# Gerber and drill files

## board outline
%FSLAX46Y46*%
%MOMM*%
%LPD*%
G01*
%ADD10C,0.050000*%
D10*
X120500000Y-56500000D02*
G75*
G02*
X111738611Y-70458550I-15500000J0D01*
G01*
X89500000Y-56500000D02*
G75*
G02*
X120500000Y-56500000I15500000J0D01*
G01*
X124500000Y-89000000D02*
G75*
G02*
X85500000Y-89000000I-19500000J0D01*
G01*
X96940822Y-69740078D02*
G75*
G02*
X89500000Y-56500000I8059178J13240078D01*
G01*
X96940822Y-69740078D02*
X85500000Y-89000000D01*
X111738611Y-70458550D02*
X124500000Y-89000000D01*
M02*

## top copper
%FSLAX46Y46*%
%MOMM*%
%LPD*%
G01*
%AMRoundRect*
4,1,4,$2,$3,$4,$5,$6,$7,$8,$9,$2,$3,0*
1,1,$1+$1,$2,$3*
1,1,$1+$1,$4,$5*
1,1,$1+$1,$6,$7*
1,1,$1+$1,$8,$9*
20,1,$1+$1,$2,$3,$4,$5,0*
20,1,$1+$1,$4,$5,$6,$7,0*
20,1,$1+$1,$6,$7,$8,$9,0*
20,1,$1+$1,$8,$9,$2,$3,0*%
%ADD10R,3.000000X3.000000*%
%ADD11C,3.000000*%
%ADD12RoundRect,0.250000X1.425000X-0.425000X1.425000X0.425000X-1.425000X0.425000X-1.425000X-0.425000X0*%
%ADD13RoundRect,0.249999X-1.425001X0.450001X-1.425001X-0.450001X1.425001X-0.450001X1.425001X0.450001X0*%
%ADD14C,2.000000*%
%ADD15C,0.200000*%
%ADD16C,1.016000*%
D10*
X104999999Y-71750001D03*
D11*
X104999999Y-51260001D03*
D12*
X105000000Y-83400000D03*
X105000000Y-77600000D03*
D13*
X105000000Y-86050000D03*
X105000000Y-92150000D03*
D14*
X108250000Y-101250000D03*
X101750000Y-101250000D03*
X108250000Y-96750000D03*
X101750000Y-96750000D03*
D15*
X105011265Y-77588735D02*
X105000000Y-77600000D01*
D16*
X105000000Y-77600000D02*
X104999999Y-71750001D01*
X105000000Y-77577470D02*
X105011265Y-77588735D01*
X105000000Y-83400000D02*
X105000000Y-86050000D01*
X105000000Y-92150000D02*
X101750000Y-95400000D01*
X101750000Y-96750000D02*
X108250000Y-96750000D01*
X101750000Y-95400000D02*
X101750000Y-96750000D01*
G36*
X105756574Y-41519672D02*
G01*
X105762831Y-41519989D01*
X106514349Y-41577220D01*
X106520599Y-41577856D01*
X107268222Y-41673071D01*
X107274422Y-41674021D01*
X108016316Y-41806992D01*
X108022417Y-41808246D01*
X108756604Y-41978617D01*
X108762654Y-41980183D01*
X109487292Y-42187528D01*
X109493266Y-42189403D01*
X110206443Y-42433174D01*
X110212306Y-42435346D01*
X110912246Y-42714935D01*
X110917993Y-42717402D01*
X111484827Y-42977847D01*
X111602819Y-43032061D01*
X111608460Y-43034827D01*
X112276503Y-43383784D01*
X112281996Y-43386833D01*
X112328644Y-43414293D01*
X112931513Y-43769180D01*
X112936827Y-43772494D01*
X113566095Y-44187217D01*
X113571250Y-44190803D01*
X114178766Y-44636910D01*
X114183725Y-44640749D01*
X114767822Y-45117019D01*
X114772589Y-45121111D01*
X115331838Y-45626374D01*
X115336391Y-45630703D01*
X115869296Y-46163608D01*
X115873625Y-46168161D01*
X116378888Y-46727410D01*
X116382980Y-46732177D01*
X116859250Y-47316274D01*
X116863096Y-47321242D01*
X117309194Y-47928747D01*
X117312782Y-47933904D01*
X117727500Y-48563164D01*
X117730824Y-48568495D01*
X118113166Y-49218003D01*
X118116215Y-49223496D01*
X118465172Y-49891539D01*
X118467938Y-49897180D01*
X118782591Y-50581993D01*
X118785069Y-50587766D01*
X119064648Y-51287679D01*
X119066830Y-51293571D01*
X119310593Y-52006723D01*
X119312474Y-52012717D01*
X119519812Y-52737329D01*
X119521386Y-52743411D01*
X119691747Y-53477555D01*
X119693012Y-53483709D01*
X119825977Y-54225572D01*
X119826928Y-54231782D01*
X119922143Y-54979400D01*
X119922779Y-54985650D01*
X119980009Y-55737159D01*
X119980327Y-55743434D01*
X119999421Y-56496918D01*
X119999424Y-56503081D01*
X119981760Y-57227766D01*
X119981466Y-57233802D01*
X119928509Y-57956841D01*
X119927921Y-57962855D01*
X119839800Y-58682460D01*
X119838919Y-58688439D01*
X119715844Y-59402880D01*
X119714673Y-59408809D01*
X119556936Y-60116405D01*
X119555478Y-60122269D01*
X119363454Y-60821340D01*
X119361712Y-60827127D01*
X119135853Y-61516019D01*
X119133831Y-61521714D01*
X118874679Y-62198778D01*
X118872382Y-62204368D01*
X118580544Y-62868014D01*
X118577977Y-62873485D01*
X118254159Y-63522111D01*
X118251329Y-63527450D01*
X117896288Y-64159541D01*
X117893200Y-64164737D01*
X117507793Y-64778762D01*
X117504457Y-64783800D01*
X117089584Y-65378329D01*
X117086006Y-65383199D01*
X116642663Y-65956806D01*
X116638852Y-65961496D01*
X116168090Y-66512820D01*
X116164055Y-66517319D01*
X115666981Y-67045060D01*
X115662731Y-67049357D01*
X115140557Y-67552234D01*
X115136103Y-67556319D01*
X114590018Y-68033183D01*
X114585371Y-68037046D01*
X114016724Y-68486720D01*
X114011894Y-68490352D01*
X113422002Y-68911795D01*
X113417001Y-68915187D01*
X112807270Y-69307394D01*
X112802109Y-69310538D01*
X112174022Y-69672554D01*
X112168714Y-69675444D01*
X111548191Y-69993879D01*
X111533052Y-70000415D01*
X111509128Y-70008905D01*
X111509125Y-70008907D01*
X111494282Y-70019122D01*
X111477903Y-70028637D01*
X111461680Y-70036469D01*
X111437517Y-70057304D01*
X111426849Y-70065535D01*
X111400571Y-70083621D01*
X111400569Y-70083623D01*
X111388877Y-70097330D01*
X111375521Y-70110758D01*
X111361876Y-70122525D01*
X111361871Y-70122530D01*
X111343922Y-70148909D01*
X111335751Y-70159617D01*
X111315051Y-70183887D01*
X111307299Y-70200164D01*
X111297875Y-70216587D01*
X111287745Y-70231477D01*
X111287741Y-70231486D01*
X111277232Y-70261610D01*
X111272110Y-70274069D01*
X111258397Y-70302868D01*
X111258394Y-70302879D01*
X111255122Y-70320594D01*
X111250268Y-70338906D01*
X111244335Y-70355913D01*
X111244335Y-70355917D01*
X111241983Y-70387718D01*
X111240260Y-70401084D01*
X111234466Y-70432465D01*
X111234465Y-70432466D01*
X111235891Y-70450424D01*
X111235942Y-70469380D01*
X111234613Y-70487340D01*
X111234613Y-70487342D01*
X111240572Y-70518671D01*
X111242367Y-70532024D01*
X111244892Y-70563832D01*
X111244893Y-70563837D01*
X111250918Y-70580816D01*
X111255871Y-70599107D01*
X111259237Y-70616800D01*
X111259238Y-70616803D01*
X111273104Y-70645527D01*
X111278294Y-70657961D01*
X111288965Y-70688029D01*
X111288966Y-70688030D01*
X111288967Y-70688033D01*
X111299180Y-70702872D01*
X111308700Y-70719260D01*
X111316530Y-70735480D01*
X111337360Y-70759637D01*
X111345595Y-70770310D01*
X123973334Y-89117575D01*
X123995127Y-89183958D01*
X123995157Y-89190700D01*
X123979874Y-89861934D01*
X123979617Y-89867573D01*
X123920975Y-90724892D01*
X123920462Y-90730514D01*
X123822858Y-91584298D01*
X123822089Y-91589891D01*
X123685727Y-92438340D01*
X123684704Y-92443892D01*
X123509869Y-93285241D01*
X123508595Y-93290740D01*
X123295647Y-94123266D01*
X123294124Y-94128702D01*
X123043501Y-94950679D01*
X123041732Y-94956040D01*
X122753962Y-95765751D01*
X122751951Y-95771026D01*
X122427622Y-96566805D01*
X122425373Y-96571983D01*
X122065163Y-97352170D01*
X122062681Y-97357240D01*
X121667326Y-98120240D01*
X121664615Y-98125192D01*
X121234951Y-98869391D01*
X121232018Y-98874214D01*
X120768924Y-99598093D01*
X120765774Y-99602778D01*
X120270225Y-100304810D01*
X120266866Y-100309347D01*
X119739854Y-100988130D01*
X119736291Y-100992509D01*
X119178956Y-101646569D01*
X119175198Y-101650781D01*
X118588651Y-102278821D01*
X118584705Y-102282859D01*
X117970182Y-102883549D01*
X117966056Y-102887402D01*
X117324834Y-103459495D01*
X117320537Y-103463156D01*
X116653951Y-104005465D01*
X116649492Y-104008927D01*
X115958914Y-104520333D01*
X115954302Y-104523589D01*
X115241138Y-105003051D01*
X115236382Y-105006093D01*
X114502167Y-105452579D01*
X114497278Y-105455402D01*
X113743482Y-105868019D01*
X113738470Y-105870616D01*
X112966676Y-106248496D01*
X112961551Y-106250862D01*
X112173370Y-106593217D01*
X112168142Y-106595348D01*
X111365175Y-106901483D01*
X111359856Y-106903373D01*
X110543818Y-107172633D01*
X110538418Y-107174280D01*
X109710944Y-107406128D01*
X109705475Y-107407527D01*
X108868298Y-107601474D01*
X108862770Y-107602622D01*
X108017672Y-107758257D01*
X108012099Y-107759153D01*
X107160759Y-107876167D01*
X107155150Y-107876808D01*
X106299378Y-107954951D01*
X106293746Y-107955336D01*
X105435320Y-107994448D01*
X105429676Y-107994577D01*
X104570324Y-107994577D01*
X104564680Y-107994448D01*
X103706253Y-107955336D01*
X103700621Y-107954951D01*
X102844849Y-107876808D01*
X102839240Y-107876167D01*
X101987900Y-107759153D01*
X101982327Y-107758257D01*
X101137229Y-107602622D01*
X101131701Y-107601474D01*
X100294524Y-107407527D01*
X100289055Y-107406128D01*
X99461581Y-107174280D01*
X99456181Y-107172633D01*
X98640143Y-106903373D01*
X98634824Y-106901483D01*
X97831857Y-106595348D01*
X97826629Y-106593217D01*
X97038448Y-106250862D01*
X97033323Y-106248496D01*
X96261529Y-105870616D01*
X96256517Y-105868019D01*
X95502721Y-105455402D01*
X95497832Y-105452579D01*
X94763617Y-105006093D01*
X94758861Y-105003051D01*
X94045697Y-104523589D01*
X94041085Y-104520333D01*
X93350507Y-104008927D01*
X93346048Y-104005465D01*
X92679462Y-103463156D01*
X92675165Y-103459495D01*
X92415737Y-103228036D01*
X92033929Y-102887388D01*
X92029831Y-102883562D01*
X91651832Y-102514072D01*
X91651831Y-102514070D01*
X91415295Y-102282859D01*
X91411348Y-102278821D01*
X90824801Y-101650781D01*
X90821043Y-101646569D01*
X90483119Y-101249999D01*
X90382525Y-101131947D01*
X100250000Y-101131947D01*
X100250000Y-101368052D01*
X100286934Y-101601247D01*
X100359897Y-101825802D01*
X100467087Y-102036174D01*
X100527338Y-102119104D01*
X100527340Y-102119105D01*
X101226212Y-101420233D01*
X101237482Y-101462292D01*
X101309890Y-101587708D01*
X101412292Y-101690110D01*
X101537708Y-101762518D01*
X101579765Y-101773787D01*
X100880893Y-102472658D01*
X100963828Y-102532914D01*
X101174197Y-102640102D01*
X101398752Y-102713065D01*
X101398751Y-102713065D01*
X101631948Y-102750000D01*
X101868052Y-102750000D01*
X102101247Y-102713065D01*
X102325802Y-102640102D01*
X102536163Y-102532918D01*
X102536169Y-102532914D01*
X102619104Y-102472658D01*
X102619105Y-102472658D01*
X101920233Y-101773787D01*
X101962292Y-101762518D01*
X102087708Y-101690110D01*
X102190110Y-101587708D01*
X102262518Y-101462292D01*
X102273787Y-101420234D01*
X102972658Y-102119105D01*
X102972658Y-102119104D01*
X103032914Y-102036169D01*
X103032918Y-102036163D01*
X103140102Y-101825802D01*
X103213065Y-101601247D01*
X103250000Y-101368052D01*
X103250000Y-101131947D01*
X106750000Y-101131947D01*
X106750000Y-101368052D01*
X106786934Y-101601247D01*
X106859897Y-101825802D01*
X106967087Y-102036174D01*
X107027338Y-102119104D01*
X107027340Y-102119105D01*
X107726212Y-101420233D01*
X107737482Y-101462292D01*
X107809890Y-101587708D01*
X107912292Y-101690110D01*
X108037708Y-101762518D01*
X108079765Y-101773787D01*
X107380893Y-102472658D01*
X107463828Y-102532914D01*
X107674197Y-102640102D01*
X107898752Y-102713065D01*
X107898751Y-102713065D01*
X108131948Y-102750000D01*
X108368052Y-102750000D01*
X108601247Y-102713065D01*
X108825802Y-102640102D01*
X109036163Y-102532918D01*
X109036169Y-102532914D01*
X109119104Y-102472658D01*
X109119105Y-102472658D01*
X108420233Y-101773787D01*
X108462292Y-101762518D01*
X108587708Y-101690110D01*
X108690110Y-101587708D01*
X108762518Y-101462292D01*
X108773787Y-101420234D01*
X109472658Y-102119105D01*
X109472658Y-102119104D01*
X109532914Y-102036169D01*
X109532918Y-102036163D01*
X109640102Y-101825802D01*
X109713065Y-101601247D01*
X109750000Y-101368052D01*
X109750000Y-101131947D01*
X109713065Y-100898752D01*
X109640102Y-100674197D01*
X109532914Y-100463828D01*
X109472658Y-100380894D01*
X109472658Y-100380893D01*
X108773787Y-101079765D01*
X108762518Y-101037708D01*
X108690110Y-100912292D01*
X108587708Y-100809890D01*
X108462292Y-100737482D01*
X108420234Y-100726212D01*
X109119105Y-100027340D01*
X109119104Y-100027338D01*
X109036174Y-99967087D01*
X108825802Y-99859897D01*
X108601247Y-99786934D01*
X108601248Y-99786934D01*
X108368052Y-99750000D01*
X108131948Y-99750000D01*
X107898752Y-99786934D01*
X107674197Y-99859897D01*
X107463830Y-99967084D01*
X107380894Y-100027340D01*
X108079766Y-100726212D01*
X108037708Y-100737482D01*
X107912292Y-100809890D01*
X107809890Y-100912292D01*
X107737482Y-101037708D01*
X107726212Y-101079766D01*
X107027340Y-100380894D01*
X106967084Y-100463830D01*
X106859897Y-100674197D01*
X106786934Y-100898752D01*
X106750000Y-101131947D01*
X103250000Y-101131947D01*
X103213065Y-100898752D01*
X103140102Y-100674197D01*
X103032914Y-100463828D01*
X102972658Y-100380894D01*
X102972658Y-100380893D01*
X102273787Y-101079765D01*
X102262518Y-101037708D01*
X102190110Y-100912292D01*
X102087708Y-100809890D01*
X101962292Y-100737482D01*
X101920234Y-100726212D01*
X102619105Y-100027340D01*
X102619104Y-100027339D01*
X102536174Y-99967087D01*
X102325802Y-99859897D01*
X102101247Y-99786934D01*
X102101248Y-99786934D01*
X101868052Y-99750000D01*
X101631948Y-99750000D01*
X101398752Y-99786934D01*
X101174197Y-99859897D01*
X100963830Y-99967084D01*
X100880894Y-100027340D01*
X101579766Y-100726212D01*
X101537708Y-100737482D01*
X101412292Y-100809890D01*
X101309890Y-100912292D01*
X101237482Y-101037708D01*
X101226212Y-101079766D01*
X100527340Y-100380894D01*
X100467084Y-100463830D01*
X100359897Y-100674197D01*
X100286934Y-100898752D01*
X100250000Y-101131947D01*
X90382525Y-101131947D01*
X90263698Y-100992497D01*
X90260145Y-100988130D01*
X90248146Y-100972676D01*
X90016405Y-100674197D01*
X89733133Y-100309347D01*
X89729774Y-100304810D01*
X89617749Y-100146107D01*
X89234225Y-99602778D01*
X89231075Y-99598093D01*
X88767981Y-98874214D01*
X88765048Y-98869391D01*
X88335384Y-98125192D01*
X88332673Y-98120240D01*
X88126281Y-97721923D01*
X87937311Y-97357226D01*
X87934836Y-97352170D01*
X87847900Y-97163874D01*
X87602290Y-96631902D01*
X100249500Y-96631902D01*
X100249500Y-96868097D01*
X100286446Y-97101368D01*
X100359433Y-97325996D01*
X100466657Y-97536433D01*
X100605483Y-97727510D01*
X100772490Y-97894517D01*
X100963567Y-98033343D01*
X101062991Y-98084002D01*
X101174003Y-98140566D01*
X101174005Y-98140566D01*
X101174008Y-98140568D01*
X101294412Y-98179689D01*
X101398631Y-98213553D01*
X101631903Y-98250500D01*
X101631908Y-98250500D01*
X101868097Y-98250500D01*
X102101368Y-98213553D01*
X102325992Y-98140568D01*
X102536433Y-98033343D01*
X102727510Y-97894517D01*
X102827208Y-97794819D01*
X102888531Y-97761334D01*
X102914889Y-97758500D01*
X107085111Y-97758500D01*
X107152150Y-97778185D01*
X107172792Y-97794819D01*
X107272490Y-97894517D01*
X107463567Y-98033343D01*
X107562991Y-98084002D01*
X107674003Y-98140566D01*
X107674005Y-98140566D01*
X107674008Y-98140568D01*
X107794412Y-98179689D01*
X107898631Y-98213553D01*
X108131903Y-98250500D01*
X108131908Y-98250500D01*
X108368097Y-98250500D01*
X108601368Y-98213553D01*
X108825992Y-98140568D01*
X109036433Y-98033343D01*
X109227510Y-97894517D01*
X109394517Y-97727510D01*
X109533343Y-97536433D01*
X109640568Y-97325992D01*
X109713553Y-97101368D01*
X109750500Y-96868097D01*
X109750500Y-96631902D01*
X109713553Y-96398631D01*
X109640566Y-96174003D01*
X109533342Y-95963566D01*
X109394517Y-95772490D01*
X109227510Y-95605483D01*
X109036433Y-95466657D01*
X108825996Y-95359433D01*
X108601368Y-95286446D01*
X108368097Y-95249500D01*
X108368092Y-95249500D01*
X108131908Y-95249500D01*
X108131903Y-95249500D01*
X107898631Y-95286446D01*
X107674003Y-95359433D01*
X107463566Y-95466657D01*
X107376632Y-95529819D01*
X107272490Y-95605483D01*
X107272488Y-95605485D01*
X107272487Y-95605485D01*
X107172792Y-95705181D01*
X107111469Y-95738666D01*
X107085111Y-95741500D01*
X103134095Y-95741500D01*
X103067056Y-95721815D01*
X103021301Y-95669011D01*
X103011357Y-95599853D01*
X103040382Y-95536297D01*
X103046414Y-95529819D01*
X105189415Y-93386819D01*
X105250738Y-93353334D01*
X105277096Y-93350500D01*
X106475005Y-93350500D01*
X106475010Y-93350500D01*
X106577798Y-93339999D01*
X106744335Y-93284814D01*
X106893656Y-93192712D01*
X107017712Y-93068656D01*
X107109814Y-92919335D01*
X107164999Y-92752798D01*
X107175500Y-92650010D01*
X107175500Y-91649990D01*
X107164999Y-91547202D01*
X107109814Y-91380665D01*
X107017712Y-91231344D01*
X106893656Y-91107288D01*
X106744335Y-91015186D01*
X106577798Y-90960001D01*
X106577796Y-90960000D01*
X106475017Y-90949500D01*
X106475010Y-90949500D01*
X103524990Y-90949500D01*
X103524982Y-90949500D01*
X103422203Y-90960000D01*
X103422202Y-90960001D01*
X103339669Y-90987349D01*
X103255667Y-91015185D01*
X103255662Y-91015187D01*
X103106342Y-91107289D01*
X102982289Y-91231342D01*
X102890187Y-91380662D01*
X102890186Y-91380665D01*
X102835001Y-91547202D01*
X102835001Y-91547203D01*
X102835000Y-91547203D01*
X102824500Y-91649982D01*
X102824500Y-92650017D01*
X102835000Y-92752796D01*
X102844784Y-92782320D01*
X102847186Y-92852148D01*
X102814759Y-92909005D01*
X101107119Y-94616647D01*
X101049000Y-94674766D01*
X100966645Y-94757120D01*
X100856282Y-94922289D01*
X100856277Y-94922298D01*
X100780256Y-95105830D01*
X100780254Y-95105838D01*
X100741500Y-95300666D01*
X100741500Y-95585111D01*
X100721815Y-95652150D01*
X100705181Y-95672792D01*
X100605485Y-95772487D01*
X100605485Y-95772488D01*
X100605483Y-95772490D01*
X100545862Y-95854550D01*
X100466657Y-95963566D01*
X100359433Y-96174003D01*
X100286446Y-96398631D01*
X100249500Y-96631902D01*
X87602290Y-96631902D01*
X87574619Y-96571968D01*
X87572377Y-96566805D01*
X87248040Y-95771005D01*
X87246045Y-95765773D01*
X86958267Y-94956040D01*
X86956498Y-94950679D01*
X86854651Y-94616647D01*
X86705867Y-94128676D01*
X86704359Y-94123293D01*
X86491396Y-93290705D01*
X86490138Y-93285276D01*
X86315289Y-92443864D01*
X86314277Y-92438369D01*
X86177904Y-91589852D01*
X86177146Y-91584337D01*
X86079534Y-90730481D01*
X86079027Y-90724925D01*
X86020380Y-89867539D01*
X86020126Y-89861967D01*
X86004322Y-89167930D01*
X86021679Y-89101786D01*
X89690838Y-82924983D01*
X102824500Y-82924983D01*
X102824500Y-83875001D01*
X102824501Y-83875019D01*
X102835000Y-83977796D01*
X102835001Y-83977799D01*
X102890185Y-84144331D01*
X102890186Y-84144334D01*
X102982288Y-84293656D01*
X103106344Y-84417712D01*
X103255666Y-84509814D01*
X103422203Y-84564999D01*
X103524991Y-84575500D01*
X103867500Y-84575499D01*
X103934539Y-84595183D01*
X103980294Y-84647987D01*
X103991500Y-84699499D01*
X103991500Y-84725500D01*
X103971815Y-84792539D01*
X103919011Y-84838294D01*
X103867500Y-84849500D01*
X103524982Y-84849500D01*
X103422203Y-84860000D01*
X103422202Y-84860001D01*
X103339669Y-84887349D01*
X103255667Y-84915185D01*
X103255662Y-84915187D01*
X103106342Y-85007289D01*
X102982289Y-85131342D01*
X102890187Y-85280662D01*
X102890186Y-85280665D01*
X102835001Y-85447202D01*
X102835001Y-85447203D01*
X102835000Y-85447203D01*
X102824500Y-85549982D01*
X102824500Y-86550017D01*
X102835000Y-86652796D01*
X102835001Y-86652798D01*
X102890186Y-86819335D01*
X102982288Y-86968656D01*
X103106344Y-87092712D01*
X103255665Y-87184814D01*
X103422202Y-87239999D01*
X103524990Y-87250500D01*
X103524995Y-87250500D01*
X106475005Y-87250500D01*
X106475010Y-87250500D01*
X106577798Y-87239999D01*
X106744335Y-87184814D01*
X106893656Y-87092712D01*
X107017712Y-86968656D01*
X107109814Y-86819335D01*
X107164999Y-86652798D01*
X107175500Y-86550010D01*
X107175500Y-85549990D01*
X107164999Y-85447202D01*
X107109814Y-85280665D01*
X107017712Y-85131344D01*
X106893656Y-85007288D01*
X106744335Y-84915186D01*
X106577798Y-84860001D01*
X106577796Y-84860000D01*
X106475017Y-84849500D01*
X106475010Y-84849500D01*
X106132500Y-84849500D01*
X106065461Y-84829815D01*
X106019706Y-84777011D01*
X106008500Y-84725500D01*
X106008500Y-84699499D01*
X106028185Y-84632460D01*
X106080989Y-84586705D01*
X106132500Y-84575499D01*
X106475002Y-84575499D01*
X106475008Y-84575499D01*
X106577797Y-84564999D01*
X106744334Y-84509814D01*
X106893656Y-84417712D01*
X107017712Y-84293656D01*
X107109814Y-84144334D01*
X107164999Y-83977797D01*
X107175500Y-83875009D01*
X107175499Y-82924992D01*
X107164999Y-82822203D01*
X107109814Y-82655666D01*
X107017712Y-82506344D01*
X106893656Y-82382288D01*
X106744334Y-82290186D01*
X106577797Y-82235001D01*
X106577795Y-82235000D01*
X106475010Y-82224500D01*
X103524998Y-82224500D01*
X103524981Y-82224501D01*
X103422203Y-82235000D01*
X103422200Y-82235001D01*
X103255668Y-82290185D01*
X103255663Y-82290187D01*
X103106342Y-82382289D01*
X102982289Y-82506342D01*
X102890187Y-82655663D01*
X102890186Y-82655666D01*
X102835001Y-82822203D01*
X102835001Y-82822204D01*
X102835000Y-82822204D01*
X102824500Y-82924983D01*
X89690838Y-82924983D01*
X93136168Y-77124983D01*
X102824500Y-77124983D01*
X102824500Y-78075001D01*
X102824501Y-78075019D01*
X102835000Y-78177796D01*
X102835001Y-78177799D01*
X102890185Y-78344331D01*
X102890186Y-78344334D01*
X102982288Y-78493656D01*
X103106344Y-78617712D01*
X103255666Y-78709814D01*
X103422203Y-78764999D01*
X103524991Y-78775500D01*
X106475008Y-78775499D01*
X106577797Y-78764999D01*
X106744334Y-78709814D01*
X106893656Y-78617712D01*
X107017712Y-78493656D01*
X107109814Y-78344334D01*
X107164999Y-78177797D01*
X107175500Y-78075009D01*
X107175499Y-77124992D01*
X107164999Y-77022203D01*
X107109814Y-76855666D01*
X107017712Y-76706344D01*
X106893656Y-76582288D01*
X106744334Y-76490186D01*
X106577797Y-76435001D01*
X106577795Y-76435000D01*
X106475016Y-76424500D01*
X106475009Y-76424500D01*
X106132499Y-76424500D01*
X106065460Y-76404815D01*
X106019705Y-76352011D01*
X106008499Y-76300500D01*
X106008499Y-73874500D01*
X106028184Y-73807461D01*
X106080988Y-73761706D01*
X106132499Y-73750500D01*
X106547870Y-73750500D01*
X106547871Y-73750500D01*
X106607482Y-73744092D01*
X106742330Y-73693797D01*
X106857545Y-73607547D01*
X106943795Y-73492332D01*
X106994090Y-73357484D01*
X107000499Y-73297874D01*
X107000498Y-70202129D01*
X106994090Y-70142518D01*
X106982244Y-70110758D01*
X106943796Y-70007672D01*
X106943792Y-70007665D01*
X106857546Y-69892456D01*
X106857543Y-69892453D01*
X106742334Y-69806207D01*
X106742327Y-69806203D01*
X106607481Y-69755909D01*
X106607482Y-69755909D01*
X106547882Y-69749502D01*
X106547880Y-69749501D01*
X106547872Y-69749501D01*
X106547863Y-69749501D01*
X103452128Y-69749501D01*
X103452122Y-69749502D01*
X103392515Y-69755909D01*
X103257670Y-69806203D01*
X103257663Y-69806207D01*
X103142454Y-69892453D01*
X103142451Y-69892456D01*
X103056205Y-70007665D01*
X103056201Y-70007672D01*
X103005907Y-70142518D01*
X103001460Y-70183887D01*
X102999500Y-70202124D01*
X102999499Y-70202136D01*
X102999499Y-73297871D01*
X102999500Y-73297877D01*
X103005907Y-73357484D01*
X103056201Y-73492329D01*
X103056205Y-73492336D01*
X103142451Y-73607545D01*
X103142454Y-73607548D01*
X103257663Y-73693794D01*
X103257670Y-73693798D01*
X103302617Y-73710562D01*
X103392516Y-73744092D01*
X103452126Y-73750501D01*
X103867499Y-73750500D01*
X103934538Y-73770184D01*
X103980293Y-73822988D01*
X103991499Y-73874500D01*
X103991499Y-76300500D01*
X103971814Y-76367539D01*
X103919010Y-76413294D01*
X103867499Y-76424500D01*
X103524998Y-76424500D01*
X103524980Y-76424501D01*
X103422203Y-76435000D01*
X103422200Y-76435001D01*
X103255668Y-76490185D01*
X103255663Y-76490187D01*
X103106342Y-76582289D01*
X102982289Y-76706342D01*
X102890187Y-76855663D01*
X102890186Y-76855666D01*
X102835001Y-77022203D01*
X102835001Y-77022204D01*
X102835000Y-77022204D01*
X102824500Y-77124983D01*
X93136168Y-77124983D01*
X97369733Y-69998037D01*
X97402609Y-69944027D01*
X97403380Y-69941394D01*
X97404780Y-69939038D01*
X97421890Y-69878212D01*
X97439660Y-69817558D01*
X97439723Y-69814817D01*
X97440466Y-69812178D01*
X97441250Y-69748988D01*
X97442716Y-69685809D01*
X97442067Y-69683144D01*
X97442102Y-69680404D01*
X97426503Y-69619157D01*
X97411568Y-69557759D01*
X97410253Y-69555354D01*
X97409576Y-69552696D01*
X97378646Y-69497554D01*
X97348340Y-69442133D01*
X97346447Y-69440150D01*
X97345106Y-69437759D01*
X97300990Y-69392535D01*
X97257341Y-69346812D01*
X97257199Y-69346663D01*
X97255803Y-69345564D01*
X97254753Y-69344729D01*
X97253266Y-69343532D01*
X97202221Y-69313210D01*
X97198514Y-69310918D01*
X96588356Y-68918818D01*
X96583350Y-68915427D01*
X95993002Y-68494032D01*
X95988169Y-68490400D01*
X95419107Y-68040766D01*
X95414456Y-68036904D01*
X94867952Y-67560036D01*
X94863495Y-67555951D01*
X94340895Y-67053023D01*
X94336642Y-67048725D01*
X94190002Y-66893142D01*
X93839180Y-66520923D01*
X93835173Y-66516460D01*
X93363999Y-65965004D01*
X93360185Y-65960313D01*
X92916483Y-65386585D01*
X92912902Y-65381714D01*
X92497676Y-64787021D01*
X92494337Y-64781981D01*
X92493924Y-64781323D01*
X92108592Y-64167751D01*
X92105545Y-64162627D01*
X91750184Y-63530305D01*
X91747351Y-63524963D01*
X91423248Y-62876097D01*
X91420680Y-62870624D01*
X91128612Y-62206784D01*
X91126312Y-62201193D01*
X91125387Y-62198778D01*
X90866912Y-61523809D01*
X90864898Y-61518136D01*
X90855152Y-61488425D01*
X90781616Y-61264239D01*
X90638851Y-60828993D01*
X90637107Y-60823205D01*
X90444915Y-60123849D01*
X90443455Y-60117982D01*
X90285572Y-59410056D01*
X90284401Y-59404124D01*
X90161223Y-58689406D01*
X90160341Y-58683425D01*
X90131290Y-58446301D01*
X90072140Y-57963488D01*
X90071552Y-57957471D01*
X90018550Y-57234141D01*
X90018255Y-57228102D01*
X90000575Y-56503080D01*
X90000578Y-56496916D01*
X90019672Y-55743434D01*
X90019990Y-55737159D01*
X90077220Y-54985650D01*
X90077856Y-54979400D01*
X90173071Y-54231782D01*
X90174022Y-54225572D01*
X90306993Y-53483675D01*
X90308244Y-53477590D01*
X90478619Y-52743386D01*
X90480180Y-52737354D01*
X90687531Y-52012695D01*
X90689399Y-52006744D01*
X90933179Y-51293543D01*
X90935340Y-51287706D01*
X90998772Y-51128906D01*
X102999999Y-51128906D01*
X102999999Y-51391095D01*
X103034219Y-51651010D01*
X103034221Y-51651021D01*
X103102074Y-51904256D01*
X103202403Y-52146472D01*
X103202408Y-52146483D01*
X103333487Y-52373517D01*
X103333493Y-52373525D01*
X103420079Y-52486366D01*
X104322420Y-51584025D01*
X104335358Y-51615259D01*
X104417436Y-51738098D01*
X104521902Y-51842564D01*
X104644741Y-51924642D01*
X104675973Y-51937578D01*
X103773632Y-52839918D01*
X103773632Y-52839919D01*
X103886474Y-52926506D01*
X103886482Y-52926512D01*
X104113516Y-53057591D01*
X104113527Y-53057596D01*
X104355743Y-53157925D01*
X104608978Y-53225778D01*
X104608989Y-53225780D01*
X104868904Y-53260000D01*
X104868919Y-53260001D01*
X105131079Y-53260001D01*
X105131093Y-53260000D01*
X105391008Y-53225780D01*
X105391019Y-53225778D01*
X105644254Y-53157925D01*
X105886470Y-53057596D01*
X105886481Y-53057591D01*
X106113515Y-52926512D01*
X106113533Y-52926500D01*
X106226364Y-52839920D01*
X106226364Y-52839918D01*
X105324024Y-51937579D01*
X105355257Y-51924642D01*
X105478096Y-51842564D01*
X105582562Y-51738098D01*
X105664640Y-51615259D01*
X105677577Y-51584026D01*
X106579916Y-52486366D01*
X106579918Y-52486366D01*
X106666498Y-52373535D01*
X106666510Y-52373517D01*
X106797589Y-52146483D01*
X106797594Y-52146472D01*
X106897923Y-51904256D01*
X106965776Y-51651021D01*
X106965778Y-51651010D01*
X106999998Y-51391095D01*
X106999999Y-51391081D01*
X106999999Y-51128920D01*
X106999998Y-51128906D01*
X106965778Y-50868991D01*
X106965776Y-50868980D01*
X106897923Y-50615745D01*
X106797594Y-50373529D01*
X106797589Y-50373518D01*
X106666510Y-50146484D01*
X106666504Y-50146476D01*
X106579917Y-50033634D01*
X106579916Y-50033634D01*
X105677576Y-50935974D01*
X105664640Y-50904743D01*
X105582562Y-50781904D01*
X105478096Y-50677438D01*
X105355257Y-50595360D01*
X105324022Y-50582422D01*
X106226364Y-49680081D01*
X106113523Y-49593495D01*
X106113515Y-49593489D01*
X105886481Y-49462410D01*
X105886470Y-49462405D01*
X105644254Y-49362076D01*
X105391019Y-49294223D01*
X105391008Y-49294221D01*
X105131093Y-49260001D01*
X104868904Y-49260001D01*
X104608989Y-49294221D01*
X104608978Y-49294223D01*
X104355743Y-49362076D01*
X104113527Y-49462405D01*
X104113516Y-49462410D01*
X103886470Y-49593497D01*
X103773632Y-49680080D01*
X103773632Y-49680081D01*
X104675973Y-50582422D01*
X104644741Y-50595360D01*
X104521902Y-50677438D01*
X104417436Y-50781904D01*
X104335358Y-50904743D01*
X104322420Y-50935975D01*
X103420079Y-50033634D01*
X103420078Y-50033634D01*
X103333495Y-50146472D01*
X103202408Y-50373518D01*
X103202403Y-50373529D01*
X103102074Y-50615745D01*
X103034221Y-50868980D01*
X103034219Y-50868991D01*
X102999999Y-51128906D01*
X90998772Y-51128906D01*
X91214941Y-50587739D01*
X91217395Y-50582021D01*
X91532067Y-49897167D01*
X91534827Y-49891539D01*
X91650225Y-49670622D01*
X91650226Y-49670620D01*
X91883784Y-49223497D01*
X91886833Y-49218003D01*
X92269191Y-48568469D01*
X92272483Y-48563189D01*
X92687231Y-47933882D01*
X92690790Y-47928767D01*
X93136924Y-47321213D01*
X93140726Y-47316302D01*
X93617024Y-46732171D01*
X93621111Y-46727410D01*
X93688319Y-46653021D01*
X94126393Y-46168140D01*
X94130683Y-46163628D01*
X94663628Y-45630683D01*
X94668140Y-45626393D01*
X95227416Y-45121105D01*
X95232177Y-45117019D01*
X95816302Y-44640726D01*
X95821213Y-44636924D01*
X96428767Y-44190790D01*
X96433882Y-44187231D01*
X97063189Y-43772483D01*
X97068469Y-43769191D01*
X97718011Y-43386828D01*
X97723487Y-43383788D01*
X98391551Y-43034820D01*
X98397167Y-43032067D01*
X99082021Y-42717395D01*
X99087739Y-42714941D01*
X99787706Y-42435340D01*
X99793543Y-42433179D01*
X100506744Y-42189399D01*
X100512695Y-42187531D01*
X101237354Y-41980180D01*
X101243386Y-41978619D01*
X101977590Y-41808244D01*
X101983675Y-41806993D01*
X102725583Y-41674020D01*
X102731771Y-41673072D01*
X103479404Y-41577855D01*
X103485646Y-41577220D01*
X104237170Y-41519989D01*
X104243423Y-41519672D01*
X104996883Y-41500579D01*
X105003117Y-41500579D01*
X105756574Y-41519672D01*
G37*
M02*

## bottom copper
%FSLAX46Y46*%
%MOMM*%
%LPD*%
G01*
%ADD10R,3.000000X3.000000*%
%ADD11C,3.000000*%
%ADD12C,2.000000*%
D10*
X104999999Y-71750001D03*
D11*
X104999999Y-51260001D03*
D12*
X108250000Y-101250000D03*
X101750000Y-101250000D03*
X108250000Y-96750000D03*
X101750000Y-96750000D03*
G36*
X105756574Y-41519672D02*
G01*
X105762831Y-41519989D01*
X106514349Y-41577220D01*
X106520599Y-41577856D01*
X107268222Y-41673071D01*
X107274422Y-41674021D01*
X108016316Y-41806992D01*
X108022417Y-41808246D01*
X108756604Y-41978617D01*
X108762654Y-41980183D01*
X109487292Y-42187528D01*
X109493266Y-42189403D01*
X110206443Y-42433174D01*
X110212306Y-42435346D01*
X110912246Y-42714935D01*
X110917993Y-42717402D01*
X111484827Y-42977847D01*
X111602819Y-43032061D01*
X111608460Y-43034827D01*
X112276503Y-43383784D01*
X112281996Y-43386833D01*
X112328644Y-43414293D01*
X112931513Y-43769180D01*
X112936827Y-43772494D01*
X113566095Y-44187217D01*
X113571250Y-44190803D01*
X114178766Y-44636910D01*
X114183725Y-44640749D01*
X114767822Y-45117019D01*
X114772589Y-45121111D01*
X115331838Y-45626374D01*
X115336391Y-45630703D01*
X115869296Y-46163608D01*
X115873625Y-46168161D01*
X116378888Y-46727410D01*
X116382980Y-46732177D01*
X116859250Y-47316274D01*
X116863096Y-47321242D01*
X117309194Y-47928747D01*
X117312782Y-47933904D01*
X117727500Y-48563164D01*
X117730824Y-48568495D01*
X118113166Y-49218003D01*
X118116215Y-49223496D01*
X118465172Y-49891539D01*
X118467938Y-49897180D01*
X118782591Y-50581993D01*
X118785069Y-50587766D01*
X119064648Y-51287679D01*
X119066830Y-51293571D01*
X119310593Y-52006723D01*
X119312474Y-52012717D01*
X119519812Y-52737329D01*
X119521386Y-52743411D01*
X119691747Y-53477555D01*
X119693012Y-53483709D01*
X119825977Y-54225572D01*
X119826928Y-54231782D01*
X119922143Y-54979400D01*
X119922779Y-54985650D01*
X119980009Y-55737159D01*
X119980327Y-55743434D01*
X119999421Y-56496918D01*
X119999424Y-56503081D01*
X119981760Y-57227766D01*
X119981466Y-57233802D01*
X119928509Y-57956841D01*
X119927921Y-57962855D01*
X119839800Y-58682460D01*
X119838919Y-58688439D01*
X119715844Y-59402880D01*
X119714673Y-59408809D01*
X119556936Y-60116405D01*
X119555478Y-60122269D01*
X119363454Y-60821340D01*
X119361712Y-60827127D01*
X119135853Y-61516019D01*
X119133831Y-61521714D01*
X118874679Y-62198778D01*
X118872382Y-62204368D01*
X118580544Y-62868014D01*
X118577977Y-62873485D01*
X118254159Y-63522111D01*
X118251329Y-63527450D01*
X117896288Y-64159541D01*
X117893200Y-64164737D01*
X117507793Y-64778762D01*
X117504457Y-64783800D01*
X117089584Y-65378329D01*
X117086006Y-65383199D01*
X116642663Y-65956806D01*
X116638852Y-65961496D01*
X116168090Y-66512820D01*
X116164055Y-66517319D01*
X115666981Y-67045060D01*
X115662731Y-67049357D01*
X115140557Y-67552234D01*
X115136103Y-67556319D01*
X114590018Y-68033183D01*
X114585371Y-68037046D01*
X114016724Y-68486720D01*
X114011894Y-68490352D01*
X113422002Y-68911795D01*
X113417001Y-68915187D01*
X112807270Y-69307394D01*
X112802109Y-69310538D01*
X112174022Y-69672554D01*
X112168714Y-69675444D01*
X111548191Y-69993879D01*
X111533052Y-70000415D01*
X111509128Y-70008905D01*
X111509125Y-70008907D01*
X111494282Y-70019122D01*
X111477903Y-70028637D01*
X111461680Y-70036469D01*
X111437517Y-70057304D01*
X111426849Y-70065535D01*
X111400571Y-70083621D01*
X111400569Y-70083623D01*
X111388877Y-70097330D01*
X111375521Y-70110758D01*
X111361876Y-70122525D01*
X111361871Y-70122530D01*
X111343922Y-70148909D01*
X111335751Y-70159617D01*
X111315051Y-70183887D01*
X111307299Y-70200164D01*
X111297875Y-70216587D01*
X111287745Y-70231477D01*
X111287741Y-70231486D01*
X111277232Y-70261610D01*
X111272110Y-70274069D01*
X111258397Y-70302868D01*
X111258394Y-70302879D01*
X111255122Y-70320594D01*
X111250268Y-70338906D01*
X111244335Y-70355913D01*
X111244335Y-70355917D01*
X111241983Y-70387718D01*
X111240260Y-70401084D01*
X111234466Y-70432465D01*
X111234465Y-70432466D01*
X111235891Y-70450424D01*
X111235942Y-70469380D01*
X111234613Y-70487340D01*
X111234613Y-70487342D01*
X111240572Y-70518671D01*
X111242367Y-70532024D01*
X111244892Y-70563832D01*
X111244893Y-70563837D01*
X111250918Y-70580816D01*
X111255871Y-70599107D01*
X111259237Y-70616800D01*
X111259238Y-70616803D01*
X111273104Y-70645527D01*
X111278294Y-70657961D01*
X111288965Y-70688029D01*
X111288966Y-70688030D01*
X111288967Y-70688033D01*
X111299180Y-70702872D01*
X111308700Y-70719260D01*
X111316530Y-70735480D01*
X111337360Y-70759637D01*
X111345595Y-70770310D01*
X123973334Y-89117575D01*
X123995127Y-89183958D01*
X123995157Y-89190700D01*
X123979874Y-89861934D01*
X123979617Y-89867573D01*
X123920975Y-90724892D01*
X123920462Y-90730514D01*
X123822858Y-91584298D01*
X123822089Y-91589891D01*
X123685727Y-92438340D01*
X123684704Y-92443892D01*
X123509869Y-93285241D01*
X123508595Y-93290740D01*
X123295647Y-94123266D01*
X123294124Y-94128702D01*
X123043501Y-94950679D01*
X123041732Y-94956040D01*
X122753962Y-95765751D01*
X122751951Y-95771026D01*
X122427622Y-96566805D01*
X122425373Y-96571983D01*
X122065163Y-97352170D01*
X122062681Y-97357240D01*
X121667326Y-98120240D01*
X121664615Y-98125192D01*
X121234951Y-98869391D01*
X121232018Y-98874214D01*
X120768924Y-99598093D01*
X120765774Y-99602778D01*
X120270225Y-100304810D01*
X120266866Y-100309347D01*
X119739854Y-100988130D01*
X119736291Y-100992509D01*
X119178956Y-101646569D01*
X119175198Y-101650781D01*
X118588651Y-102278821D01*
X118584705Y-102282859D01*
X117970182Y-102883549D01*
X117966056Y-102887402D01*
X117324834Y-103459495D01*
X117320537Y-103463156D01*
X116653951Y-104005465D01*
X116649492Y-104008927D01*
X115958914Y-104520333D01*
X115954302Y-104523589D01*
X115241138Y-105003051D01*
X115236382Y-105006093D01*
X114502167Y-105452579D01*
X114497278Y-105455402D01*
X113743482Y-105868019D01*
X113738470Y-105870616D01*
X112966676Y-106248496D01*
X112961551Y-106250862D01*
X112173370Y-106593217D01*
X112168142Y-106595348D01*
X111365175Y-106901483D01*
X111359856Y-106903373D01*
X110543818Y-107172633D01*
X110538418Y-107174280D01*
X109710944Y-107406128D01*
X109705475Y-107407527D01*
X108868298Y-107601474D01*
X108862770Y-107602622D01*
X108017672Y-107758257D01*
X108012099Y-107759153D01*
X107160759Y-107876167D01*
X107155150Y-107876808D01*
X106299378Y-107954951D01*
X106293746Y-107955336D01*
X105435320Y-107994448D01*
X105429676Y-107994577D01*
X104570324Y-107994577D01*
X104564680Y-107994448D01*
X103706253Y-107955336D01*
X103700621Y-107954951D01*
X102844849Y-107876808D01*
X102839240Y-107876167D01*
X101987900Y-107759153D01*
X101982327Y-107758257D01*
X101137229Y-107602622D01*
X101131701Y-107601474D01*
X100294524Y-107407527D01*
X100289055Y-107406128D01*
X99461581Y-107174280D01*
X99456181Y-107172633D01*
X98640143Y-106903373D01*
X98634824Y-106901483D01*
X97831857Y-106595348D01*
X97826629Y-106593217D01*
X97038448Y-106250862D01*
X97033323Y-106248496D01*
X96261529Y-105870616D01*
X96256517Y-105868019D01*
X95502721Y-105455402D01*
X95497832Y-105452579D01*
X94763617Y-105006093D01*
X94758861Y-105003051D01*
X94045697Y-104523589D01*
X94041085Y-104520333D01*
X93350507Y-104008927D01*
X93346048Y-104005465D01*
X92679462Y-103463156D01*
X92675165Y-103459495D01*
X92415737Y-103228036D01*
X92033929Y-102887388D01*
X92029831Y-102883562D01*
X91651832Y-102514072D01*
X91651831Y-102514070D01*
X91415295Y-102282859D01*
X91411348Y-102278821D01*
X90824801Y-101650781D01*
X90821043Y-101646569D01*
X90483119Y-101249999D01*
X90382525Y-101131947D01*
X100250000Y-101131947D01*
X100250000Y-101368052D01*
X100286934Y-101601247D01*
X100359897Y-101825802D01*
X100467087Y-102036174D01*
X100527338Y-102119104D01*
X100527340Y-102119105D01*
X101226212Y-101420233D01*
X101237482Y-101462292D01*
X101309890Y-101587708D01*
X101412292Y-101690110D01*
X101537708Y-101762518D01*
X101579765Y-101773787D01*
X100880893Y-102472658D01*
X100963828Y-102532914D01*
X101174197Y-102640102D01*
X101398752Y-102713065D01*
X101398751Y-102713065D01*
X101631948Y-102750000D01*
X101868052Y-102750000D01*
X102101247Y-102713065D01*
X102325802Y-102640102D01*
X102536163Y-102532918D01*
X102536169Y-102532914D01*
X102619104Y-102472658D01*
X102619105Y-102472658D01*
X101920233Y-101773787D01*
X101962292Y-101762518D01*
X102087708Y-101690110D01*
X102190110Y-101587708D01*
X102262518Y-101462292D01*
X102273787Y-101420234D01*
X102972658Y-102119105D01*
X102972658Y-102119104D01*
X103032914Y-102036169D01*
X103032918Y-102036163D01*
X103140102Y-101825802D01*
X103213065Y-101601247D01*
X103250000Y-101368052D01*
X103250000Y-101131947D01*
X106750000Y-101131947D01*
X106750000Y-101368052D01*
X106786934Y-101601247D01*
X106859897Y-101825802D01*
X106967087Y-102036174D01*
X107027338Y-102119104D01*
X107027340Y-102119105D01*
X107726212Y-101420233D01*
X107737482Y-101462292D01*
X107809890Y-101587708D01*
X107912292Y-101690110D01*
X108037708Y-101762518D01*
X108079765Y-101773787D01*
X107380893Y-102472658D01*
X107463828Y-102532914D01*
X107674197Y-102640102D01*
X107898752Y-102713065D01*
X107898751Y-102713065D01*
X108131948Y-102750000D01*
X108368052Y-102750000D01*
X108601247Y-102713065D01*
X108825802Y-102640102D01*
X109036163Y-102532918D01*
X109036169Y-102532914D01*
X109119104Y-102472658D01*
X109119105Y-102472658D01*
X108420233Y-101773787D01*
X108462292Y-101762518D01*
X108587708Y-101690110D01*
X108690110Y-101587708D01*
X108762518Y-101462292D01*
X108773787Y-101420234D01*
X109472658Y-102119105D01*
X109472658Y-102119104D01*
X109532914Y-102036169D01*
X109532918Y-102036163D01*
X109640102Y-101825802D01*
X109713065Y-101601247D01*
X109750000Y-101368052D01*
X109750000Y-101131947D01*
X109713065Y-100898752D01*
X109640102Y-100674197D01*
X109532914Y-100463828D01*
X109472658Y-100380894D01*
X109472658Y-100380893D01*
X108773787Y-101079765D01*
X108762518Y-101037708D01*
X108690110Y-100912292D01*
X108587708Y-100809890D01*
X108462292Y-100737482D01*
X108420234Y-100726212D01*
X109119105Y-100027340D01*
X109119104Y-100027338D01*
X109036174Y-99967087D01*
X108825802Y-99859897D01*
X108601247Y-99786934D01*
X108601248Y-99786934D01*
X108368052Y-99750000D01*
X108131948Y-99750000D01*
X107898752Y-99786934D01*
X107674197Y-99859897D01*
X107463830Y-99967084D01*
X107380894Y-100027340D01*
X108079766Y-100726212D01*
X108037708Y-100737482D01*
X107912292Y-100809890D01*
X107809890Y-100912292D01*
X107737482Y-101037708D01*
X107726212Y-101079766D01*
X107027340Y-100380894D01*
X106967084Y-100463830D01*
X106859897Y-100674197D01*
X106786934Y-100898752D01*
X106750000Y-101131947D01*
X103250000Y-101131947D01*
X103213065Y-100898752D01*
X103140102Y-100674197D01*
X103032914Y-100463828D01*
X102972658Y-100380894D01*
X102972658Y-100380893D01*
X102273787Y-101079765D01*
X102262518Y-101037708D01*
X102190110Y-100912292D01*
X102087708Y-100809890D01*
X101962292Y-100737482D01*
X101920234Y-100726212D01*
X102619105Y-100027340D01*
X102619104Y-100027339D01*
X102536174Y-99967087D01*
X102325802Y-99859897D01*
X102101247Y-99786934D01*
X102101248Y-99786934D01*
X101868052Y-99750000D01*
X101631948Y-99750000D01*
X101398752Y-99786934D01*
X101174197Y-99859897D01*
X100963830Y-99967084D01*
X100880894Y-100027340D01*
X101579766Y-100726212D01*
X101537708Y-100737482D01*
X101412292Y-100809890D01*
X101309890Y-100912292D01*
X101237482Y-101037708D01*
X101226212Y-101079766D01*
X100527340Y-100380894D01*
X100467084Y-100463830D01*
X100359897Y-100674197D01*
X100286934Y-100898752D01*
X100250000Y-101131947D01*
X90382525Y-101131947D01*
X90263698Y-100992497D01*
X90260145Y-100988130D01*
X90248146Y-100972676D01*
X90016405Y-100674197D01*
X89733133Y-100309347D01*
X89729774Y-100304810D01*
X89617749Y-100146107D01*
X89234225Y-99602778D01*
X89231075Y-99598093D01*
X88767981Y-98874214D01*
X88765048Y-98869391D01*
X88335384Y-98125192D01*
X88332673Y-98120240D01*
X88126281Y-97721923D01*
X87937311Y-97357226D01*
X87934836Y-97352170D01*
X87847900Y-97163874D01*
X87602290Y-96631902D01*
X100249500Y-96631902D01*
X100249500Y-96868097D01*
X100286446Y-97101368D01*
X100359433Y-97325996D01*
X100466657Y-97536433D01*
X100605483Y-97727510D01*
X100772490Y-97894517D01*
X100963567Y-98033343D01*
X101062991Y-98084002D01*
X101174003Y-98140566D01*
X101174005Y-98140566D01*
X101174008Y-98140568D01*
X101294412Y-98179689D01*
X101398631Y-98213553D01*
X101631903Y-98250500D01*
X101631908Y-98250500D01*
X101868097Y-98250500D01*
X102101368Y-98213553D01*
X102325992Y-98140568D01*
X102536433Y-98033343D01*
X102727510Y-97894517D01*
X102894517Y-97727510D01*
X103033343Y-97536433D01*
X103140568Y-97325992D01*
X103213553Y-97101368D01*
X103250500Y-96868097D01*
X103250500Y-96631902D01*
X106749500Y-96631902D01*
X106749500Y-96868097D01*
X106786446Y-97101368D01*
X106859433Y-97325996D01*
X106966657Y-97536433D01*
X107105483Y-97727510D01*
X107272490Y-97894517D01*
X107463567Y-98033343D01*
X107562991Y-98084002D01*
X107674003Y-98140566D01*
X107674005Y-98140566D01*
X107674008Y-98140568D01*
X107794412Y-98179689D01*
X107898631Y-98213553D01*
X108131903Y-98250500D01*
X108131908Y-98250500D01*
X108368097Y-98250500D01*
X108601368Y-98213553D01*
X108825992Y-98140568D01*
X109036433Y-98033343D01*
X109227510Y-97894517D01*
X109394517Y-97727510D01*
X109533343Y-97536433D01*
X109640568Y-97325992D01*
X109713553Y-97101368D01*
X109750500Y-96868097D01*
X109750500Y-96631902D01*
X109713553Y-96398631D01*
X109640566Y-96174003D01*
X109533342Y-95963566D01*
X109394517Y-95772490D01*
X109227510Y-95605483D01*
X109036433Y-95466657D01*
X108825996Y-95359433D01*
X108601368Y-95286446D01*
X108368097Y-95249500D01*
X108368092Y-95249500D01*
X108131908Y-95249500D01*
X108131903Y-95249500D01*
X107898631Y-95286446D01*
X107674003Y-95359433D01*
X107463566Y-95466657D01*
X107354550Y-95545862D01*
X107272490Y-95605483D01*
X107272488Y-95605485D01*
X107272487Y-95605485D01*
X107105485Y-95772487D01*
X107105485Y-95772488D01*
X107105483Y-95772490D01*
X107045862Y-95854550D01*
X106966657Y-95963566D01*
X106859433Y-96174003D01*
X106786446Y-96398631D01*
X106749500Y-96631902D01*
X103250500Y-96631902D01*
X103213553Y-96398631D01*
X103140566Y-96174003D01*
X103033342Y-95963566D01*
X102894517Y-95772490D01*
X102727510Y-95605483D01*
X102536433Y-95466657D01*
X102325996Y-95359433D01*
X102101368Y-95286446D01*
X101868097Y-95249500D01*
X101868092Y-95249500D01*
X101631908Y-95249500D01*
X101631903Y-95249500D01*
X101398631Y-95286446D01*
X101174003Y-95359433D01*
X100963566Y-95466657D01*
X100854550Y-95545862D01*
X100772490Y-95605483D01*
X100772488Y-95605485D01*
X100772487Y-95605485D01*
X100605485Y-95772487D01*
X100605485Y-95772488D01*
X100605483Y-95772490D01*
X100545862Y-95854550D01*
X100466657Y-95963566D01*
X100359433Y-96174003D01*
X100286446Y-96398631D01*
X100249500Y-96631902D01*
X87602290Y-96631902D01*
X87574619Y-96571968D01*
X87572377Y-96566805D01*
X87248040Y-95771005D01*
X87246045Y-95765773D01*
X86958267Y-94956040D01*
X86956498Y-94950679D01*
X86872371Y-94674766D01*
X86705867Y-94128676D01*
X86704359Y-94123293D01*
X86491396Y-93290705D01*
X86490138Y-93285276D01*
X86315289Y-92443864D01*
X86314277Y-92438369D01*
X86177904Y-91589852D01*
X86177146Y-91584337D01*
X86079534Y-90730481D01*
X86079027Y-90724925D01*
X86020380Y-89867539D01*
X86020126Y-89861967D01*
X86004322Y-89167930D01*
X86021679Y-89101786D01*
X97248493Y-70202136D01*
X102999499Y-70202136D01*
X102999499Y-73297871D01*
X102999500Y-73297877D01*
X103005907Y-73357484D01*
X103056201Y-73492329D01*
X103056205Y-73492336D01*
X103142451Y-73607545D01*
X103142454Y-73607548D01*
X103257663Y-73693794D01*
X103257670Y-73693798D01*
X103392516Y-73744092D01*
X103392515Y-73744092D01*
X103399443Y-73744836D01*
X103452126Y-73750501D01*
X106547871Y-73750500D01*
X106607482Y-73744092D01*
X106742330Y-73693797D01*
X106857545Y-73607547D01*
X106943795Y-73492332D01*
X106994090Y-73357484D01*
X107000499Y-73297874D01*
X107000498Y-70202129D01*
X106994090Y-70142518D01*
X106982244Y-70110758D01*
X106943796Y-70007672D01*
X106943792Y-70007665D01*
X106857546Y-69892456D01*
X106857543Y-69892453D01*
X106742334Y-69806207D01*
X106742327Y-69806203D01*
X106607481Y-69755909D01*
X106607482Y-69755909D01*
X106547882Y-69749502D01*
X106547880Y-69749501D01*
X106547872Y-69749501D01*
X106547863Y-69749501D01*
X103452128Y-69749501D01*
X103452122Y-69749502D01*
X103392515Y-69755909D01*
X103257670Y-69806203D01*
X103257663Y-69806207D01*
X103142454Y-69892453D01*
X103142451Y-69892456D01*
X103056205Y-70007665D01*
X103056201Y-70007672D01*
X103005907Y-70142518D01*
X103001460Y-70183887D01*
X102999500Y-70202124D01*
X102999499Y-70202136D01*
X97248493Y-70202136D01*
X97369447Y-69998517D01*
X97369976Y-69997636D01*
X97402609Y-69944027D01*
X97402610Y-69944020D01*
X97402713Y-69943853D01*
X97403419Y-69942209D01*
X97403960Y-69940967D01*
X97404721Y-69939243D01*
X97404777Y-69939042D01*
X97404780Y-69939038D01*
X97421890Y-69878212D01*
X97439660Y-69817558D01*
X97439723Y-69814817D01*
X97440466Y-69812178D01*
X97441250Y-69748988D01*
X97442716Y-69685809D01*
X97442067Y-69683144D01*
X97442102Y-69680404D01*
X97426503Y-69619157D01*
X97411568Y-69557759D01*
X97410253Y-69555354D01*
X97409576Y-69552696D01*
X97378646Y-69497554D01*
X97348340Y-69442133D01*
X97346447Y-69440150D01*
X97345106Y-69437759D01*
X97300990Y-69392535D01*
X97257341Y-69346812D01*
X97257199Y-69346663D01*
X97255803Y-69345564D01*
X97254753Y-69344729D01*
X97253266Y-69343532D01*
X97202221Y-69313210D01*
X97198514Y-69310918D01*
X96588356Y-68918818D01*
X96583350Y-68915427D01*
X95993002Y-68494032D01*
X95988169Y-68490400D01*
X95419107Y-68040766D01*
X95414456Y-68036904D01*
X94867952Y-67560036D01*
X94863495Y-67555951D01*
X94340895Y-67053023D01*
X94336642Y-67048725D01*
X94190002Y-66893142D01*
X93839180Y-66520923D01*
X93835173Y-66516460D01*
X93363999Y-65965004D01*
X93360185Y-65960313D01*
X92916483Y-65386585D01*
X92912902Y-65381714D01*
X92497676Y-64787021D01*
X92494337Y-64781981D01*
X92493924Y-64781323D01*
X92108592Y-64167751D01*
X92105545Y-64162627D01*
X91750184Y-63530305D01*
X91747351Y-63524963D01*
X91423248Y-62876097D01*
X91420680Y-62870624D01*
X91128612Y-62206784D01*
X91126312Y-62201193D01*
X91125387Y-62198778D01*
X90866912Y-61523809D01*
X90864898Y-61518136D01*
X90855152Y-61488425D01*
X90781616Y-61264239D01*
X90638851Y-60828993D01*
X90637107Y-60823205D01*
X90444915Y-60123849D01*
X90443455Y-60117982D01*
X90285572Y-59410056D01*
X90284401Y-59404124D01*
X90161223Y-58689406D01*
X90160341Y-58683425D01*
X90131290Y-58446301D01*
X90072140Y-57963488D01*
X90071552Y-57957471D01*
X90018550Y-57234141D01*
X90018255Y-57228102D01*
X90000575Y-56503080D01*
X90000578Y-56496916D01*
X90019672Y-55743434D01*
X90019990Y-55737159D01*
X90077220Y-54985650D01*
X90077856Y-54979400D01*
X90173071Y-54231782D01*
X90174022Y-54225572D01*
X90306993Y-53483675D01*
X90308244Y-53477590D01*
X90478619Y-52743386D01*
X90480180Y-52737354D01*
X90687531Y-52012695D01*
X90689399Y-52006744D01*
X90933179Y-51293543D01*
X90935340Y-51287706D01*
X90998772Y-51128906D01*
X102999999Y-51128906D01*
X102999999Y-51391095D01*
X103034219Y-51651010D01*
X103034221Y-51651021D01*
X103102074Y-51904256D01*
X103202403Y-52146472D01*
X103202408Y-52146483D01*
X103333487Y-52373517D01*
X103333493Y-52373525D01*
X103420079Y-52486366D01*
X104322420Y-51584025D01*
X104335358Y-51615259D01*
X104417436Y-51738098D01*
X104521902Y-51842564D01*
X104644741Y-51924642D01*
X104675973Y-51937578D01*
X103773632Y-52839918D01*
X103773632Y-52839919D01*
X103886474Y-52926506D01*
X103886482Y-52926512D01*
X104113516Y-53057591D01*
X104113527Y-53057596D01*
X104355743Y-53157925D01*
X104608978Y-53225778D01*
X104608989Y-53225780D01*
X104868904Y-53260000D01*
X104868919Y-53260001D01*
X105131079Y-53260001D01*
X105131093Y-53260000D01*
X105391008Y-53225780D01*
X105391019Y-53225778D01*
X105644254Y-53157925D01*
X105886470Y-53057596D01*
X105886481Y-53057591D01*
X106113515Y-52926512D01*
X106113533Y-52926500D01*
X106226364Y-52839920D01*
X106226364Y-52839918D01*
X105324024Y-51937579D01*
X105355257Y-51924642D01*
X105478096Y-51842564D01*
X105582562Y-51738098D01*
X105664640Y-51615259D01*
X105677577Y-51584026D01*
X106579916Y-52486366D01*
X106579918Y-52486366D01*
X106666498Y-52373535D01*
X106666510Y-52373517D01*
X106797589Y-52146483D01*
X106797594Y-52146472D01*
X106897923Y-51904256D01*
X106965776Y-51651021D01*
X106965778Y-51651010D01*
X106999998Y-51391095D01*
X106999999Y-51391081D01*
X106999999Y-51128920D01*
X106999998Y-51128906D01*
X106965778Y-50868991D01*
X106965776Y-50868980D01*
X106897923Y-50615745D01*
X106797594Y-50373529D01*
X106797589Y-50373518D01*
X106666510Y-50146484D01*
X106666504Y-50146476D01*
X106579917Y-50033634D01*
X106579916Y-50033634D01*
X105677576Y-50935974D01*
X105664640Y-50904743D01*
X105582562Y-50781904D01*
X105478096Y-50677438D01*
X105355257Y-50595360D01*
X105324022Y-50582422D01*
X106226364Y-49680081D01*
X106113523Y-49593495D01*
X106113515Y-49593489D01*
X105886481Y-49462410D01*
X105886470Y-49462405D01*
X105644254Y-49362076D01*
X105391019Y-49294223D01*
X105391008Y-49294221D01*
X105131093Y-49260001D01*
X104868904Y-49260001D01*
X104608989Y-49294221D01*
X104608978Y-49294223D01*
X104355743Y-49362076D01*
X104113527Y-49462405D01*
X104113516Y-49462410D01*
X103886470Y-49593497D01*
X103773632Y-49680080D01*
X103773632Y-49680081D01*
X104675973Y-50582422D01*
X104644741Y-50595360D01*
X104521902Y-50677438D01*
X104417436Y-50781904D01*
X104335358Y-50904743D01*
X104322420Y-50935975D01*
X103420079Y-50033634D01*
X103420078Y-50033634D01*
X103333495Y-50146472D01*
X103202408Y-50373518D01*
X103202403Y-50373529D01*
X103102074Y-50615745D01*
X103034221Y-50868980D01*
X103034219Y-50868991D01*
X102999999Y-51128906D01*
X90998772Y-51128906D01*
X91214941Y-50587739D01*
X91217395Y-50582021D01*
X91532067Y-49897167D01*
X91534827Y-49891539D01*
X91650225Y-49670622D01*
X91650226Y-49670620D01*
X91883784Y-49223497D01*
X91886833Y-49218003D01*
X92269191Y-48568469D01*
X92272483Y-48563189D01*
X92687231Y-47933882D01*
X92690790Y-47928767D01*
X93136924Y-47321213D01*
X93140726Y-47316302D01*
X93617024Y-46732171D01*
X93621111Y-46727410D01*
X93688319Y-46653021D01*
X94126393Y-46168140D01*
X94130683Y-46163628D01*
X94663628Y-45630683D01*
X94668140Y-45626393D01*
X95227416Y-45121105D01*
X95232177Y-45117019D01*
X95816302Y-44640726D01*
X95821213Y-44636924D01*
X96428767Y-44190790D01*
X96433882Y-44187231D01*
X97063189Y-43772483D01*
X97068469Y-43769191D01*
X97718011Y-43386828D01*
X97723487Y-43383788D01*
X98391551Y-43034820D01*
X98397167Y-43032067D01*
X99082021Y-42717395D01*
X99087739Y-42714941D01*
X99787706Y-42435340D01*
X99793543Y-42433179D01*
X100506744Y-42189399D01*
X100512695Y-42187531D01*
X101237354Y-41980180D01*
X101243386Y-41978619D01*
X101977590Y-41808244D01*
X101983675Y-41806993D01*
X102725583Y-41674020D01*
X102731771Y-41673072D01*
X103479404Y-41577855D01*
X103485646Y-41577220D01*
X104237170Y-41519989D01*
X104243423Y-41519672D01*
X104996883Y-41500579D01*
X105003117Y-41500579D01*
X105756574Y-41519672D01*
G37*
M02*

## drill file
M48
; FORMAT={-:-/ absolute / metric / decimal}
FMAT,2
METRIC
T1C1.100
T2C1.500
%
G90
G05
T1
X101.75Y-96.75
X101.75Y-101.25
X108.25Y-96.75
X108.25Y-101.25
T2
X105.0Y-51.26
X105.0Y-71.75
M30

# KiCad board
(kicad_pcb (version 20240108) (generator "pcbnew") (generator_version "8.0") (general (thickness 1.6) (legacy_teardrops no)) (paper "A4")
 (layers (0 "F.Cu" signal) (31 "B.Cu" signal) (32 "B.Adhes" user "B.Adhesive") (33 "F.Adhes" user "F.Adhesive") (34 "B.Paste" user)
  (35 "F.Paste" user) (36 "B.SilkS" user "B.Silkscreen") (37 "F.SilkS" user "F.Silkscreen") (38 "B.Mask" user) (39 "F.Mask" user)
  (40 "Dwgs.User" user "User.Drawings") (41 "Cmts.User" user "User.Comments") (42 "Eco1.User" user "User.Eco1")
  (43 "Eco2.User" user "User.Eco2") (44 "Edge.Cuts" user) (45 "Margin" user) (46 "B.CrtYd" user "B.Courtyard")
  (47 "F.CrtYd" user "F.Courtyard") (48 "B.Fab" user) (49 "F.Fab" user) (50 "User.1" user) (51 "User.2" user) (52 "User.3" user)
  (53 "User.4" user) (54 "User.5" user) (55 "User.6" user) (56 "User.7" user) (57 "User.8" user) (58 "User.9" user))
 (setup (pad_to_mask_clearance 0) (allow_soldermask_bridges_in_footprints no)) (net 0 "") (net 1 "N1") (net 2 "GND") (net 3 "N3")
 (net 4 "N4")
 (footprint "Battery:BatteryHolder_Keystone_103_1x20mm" (layer "F.Cu") (at 104.999999 71.750001 90)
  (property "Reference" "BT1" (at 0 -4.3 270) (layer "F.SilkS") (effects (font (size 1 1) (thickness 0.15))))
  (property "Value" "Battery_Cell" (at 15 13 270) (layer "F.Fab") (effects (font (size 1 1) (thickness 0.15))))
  (pad "1" thru_hole rect (at 0 0 90) (size 3 3) (drill 1.5) (layers "*.Cu" "*.Mask") (remove_unused_layers no) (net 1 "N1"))
  (pad "2" thru_hole circle (at 20.49 0 90) (size 3 3) (drill 1.5) (layers "*.Cu" "*.Mask") (remove_unused_layers no) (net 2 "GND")))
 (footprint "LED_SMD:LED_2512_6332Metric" (layer "F.Cu") (at 105 80.5 90)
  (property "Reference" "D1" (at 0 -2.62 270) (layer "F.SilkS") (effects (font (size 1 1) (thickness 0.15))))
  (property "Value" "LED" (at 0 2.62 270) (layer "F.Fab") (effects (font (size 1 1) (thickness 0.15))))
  (pad "1" smd roundrect (at -2.9 0 90) (size 1.35 3.35) (layers "F.Cu" "F.Paste" "F.Mask") (roundrect_rratio 0.185185) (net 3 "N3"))
  (pad "2" smd roundrect (at 2.9 0 90) (size 1.35 3.35) (layers "F.Cu" "F.Paste" "F.Mask") (roundrect_rratio 0.185185) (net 1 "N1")))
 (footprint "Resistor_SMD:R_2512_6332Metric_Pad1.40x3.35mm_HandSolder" (layer "F.Cu") (at 105 89.1 -90)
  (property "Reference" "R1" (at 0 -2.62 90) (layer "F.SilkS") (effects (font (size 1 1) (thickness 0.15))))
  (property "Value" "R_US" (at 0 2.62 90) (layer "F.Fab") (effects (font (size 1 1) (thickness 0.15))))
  (pad "1" smd roundrect (at -3.05 0 270) (size 1.4 3.35) (layers "F.Cu" "F.Paste" "F.Mask") (roundrect_rratio 0.178571) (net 3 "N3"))
  (pad "2" smd roundrect (at 3.05 0 270) (size 1.4 3.35) (layers "F.Cu" "F.Paste" "F.Mask") (roundrect_rratio 0.178571) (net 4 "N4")))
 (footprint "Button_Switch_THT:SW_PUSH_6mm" (layer "F.Cu") (at 108.25 101.25 180)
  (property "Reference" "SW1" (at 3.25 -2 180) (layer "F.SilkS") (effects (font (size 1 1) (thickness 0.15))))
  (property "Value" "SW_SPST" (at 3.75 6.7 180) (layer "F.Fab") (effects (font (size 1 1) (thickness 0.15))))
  (pad "1" thru_hole circle (at 0 0 270) (size 2 2) (drill 1.1) (layers "*.Cu" "*.Mask") (remove_unused_layers no) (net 2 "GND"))
  (pad "1" thru_hole circle (at 6.5 0 270) (size 2 2) (drill 1.1) (layers "*.Cu" "*.Mask") (remove_unused_layers no) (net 2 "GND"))
  (pad "2" thru_hole circle (at 0 4.5 270) (size 2 2) (drill 1.1) (layers "*.Cu" "*.Mask") (remove_unused_layers no) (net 4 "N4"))
  (pad "2" thru_hole circle (at 6.5 4.5 270) (size 2 2) (drill 1.1) (layers "*.Cu" "*.Mask") (remove_unused_layers no) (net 4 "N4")))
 (gr_arc (start 120.5 56.5) (mid 118.128185 64.740192) (end 111.738611 70.45855) (stroke (width 0.05) (type default)) (layer "Edge.Cuts"))
 (gr_arc (start 89.5 56.5) (mid 105 41) (end 120.5 56.5) (stroke (width 0.05) (type default)) (layer "Edge.Cuts"))
 (gr_arc (start 124.5 89) (mid 105 108.5) (end 85.5 89) (stroke (width 0.05) (type default)) (layer "Edge.Cuts"))
 (gr_arc (start 96.940822 69.740078) (mid 91.487649 64.093838) (end 89.5 56.5) (stroke (width 0.05) (type default)) (layer "Edge.Cuts"))
 (gr_line (start 96.940822 69.740078) (end 85.5 89) (stroke (width 0.05) (type default)) (layer "Edge.Cuts"))
 (gr_line (start 111.738611 70.45855) (end 124.5 89) (stroke (width 0.05) (type default)) (layer "Edge.Cuts"))
 (segment (start 105.011265 77.588735) (end 105 77.6) (width 0.2) (layer "F.Cu") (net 1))
 (segment (start 105 77.6) (end 104.999999 71.750001) (width 1.016) (layer "F.Cu") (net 1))
 (segment (start 105 77.57747) (end 105.011265 77.588735) (width 1.016) (layer "F.Cu") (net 1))
 (segment (start 105 83.4) (end 105 86.05) (width 1.016) (layer "F.Cu") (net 3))
 (segment (start 105 92.15) (end 101.75 95.4) (width 1.016) (layer "F.Cu") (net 4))
 (segment (start 101.75 96.75) (end 108.25 96.75) (width 1.016) (layer "F.Cu") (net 4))
 (segment (start 101.75 95.4) (end 101.75 96.75) (width 1.016) (layer "F.Cu") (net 4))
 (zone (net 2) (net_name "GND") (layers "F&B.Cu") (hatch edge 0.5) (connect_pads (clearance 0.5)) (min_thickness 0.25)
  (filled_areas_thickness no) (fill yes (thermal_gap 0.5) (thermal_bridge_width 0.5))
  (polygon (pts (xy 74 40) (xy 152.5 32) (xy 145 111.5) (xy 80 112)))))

